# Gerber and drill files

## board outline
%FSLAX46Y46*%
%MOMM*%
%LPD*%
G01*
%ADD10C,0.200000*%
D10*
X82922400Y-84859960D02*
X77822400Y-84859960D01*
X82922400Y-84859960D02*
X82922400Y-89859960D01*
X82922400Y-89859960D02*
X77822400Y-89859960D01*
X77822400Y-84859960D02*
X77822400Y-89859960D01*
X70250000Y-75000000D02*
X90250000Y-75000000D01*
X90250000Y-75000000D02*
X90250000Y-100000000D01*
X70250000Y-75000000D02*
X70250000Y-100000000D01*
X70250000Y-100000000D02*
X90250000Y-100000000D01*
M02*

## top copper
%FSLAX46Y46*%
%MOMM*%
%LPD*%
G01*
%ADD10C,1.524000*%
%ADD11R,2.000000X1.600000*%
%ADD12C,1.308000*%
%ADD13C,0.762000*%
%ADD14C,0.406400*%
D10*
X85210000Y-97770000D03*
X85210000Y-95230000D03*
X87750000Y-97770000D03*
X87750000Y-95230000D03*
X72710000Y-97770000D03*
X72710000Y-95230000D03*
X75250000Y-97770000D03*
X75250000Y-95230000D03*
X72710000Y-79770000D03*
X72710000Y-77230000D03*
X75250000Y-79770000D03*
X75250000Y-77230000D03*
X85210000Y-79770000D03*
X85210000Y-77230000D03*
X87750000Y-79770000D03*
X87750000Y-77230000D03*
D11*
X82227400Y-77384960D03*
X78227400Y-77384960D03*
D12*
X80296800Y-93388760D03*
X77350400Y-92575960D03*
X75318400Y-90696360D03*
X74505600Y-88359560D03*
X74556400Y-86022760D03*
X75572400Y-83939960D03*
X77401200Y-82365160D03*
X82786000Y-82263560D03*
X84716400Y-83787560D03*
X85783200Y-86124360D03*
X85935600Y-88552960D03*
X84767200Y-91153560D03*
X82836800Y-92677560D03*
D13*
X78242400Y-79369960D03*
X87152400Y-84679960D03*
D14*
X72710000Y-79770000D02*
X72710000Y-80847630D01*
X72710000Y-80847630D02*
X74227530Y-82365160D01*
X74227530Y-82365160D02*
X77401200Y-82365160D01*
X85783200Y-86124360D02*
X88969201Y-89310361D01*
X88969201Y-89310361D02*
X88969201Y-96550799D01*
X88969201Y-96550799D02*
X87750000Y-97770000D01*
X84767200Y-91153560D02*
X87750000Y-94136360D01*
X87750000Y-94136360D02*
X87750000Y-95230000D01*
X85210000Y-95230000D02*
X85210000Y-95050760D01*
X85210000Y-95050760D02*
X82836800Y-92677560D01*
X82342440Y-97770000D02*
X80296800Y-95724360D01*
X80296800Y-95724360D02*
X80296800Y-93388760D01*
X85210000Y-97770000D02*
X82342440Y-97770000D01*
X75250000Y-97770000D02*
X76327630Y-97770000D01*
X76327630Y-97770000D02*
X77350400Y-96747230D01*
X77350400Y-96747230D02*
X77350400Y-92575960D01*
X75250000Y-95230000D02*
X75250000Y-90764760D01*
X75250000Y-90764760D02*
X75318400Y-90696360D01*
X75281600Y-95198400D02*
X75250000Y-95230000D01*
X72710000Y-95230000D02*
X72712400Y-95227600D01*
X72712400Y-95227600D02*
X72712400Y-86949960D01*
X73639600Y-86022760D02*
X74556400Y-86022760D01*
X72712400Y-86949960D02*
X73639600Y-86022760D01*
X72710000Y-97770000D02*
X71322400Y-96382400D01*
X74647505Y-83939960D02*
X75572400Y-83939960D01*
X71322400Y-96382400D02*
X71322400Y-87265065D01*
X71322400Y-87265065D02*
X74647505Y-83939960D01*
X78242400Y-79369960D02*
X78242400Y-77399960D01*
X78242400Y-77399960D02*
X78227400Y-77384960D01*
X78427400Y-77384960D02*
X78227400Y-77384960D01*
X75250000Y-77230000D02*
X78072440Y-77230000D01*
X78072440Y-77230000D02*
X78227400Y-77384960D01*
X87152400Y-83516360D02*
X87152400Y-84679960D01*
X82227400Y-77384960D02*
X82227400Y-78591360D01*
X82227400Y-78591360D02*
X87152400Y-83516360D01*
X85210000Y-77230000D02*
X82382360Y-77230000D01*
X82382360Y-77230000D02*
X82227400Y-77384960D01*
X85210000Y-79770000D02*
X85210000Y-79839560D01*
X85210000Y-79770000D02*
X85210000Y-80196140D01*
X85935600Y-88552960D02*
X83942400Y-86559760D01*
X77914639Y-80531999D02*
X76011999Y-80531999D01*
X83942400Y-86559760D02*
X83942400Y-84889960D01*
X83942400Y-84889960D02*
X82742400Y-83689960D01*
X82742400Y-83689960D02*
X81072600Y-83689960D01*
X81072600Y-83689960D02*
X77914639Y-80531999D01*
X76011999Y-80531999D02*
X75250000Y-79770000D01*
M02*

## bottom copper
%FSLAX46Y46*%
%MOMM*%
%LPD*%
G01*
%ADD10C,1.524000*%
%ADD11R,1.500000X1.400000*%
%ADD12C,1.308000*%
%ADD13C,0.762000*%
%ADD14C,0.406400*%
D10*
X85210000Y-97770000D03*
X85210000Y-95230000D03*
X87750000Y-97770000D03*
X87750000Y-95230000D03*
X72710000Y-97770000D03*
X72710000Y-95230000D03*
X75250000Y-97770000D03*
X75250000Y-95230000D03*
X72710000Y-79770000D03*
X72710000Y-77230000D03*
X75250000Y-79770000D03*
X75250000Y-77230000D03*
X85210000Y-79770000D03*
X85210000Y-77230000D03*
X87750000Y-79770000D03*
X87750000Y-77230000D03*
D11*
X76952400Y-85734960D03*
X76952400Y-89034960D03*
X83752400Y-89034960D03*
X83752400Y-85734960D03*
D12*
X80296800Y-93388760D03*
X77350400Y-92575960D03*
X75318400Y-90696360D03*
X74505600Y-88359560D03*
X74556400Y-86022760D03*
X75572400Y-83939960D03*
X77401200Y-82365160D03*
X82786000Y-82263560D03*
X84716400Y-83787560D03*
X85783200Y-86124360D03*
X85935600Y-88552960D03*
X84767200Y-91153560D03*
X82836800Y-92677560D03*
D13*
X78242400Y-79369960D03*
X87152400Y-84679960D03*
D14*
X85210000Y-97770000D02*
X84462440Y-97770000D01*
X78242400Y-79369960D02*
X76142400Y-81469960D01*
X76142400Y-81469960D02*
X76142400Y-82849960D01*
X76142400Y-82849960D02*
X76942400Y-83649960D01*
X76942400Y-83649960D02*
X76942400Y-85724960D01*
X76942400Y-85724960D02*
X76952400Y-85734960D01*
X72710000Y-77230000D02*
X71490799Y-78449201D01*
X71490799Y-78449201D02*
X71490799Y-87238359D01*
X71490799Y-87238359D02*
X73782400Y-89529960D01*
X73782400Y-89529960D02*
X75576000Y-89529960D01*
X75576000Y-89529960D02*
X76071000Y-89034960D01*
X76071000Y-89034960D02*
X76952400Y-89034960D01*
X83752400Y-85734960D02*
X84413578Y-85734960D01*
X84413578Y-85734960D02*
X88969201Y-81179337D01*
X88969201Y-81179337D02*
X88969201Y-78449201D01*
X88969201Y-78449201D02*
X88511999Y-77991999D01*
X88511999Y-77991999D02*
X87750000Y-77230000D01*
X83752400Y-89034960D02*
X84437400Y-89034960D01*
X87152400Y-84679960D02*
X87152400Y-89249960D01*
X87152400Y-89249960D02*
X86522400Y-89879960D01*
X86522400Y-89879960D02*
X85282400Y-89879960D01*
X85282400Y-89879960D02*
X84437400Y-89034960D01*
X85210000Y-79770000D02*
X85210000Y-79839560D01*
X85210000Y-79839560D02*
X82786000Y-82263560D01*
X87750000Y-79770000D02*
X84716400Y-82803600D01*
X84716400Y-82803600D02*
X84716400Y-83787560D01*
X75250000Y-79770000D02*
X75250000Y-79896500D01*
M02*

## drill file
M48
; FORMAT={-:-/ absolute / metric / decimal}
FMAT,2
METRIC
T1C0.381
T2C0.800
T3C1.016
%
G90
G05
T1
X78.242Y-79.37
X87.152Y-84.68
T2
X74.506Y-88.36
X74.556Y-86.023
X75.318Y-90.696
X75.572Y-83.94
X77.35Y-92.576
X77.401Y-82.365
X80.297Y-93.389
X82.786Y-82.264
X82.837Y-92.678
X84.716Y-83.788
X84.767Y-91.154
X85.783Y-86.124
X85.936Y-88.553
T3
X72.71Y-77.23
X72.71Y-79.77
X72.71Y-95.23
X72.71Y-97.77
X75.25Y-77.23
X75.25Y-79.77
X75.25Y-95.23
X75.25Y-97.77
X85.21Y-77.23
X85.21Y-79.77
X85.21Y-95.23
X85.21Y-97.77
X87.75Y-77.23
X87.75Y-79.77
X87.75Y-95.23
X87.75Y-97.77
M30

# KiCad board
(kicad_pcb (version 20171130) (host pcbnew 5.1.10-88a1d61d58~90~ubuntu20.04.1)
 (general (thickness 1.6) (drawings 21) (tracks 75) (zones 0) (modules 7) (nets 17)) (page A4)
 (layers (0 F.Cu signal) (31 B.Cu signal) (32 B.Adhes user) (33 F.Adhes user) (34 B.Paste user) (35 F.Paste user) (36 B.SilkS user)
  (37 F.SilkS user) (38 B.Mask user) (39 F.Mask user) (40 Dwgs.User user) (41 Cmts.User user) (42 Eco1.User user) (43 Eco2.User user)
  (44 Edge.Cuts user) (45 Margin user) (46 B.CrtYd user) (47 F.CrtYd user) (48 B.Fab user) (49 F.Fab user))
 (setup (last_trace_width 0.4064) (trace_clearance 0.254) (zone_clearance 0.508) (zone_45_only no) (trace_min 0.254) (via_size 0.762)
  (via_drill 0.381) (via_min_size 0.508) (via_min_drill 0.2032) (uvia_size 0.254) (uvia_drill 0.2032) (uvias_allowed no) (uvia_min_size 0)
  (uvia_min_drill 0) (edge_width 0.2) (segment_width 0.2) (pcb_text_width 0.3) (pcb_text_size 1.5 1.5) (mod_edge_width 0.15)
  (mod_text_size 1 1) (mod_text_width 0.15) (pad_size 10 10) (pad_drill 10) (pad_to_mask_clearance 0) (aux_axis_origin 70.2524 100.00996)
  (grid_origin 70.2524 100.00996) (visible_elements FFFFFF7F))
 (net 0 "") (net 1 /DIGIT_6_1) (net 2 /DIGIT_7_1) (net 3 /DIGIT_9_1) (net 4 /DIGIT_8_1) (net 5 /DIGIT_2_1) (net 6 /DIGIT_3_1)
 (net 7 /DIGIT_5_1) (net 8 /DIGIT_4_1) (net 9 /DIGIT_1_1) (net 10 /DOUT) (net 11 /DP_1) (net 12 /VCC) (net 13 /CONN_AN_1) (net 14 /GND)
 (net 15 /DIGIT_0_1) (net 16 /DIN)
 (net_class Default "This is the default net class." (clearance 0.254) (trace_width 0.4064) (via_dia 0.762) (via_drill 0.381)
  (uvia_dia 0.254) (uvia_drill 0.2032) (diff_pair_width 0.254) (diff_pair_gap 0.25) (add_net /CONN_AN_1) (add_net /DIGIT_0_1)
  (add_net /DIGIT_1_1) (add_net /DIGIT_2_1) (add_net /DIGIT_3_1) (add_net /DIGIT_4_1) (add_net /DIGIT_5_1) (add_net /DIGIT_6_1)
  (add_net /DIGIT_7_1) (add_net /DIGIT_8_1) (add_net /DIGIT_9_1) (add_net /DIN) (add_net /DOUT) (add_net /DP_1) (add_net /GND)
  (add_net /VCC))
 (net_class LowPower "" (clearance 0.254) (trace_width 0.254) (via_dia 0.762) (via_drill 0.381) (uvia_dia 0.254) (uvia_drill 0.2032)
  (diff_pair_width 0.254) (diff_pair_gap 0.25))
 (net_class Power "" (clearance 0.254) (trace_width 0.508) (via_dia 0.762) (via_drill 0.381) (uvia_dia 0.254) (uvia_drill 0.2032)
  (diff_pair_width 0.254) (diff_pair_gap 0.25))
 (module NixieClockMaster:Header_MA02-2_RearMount (layer F.Cu) (at 87.75 96.5)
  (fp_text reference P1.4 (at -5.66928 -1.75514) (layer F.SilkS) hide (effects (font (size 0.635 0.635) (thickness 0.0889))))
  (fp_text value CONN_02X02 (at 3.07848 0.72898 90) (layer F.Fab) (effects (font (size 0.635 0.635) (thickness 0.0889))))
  (pad 1 thru_hole circle (at -2.54 1.27) (size 1.524 1.524) (drill 1.016) (layers *.Cu *.Mask F.Paste F.SilkS) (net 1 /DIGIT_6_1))
  (pad 2 thru_hole circle (at -2.54 -1.27) (size 1.524 1.524) (drill 1.016) (layers *.Cu *.Mask F.Paste F.SilkS) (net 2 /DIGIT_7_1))
  (pad 3 thru_hole circle (at 0 1.27) (size 1.524 1.524) (drill 1.016) (layers *.Cu *.Mask F.Paste F.SilkS) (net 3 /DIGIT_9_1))
  (pad 4 thru_hole circle (at 0 -1.27) (size 1.524 1.524) (drill 1.016) (layers *.Cu *.Mask F.Paste F.SilkS) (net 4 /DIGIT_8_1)))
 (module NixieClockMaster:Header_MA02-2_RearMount (layer F.Cu) (at 75.25 96.5)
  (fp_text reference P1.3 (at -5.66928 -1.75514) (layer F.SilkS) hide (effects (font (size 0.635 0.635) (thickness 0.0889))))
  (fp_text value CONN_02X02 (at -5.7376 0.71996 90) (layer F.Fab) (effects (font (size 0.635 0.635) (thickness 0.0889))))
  (pad 1 thru_hole circle (at -2.54 1.27) (size 1.524 1.524) (drill 1.016) (layers *.Cu *.Mask F.Paste F.SilkS) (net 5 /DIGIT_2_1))
  (pad 2 thru_hole circle (at -2.54 -1.27) (size 1.524 1.524) (drill 1.016) (layers *.Cu *.Mask F.Paste F.SilkS) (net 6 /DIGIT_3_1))
  (pad 3 thru_hole circle (at 0 1.27) (size 1.524 1.524) (drill 1.016) (layers *.Cu *.Mask F.Paste F.SilkS) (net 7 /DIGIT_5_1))
  (pad 4 thru_hole circle (at 0 -1.27) (size 1.524 1.524) (drill 1.016) (layers *.Cu *.Mask F.Paste F.SilkS) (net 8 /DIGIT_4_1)))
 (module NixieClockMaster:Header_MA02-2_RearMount (layer F.Cu) (at 75.25 78.5)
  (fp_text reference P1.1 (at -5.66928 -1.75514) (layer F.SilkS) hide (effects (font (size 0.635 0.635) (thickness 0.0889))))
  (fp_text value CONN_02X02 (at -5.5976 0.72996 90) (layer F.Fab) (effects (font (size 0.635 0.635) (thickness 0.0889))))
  (pad 1 thru_hole circle (at -2.54 1.27) (size 1.524 1.524) (drill 1.016) (layers *.Cu *.Mask F.Paste F.SilkS) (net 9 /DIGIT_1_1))
  (pad 2 thru_hole circle (at -2.54 -1.27) (size 1.524 1.524) (drill 1.016) (layers *.Cu *.Mask F.Paste F.SilkS) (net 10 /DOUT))
  (pad 3 thru_hole circle (at 0 1.27) (size 1.524 1.524) (drill 1.016) (layers *.Cu *.Mask F.Paste F.SilkS) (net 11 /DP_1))
  (pad 4 thru_hole circle (at 0 -1.27) (size 1.524 1.524) (drill 1.016) (layers *.Cu *.Mask F.Paste F.SilkS) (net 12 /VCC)))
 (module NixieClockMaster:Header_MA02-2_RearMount (layer F.Cu) (at 87.75 78.5)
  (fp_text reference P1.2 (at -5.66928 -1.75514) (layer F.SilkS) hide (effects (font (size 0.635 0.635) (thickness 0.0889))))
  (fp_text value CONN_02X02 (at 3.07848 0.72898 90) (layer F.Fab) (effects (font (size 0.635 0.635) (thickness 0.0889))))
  (pad 1 thru_hole circle (at -2.54 1.27) (size 1.524 1.524) (drill 1.016) (layers *.Cu *.Mask F.Paste F.SilkS) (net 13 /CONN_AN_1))
  (pad 2 thru_hole circle (at -2.54 -1.27) (size 1.524 1.524) (drill 1.016) (layers *.Cu *.Mask F.Paste F.SilkS) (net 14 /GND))
  (pad 3 thru_hole circle (at 0 1.27) (size 1.524 1.524) (drill 1.016) (layers *.Cu *.Mask F.Paste F.SilkS) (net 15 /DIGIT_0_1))
  (pad 4 thru_hole circle (at 0 -1.27) (size 1.524 1.524) (drill 1.016) (layers *.Cu *.Mask F.Paste F.SilkS) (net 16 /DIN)))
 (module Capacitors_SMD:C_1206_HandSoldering (layer F.Cu) (at 80.2274 77.38496 180)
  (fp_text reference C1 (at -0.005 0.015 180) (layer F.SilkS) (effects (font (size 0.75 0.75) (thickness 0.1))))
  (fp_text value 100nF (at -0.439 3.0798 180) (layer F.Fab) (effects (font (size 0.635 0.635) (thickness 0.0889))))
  (pad 1 smd rect (at -2 0 180) (size 2 1.6) (layers F.Cu F.Paste F.Mask) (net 14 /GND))
  (pad 2 smd rect (at 2 0 180) (size 2 1.6) (layers F.Cu F.Paste F.Mask) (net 12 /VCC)))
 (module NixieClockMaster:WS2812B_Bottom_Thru (layer F.Cu) (at 80.3524 87.38496 90)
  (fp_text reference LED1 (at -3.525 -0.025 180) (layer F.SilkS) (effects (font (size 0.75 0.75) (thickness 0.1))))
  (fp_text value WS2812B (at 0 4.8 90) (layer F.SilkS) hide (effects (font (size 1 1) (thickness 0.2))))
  (pad 1 smd rect (at 1.65 -3.4 90) (size 1.4 1.5) (layers B.Cu B.Paste B.Mask) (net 12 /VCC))
  (pad 2 smd rect (at -1.65 -3.4 90) (size 1.4 1.5) (layers B.Cu B.Paste B.Mask) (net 10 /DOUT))
  (pad 3 smd rect (at -1.65 3.4 90) (size 1.4 1.5) (layers B.Cu B.Paste B.Mask) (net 14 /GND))
  (pad 4 smd rect (at 1.65 3.4 90) (size 1.4 1.5) (layers B.Cu B.Paste B.Mask) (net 16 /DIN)))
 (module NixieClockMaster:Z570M (layer F.Cu) (at 80.1952 87.49596 180)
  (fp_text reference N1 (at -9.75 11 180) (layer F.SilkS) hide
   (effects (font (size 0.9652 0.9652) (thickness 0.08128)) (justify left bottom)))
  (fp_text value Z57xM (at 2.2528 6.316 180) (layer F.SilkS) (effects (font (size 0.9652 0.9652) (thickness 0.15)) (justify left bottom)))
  (pad 6 thru_hole circle (at -0.1016 -5.8928 180) (size 1.308 1.308) (drill 0.8) (layers *.Cu *.Mask) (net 1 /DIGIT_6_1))
  (pad 5 thru_hole circle (at 2.8448 -5.08 180) (size 1.308 1.308) (drill 0.8) (layers *.Cu *.Mask) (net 7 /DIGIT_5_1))
  (pad 4 thru_hole circle (at 4.8768 -3.2004 180) (size 1.308 1.308) (drill 0.8) (layers *.Cu *.Mask) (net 8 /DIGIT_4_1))
  (pad N/C thru_hole circle (at 5.6896 -0.8636 180) (size 1.308 1.308) (drill 0.8) (layers *.Cu *.Mask))
  (pad 3 thru_hole circle (at 5.6388 1.4732 180) (size 1.308 1.308) (drill 0.8) (layers *.Cu *.Mask) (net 6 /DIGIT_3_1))
  (pad 2 thru_hole circle (at 4.6228 3.556 180) (size 1.308 1.308) (drill 0.8) (layers *.Cu *.Mask) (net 5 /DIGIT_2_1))
  (pad 1 thru_hole circle (at 2.794 5.1308 180) (size 1.308 1.308) (drill 0.8) (layers *.Cu *.Mask) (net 9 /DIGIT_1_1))
  (pad A thru_hole circle (at -2.5908 5.2324 180) (size 1.308 1.308) (drill 0.8) (layers *.Cu *.Mask) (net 13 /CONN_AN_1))
  (pad 0 thru_hole circle (at -4.5212 3.7084 180) (size 1.308 1.308) (drill 0.8) (layers *.Cu *.Mask) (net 15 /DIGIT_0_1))
  (pad 9 thru_hole circle (at -5.588 1.3716 180) (size 1.308 1.308) (drill 0.8) (layers *.Cu *.Mask) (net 3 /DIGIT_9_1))
  (pad RHDP thru_hole circle (at -5.7404 -1.057 180) (size 1.308 1.308) (drill 0.8) (layers *.Cu *.Mask) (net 11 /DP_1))
  (pad 8 thru_hole circle (at -4.572 -3.6576 180) (size 1.308 1.308) (drill 0.8) (layers *.Cu *.Mask) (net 4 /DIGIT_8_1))
  (pad 7 thru_hole circle (at -2.6416 -5.1816 180) (size 1.308 1.308) (drill 0.8) (layers *.Cu *.Mask) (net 2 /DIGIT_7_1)))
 (gr_line (start 82.9224 84.85996) (end 77.8224 84.85996) (layer Edge.Cuts) (width 0.2))
 (gr_line (start 82.9224 84.85996) (end 82.9224 89.85996) (layer Edge.Cuts) (width 0.2))
 (gr_line (start 82.9224 89.85996) (end 77.8224 89.85996) (layer Edge.Cuts) (width 0.2))
 (gr_line (start 77.8224 84.85996) (end 77.8224 89.85996) (layer Edge.Cuts) (width 0.2))
 (gr_line (start 70.25 75) (end 90.25 75) (layer Edge.Cuts) (width 0.2))
 (gr_line (start 90.25 75) (end 90.25 100) (layer Edge.Cuts) (width 0.2))
 (gr_line (start 70.25 75) (end 70.25 100) (layer Edge.Cuts) (width 0.2))
 (gr_line (start 70.25 100) (end 90.25 100) (layer Edge.Cuts) (width 0.2))
 (segment (start 72.71 79.77) (end 72.71 80.84763) (width 0.4064) (layer F.Cu) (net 9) (status 10))
 (segment (start 72.71 80.84763) (end 74.22753 82.36516) (width 0.4064) (layer F.Cu) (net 9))
 (segment (start 74.22753 82.36516) (end 77.4012 82.36516) (width 0.4064) (layer F.Cu) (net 9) (status 20))
 (segment (start 85.7832 86.12436) (end 88.969201 89.310361) (width 0.4064) (layer F.Cu) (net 3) (status 10))
 (segment (start 88.969201 89.310361) (end 88.969201 96.550799) (width 0.4064) (layer F.Cu) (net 3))
 (segment (start 88.969201 96.550799) (end 87.75 97.77) (width 0.4064) (layer F.Cu) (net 3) (status 20))
 (segment (start 84.7672 91.15356) (end 87.75 94.13636) (width 0.4064) (layer F.Cu) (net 4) (status 10))
 (segment (start 87.75 94.13636) (end 87.75 95.23) (width 0.4064) (layer F.Cu) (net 4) (status 20))
 (segment (start 85.21 95.23) (end 85.21 95.05076) (width 0.4064) (layer F.Cu) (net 2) (status 30))
 (segment (start 85.21 95.05076) (end 82.8368 92.67756) (width 0.4064) (layer F.Cu) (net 2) (status 30))
 (segment (start 82.34244 97.77) (end 80.2968 95.72436) (width 0.4064) (layer F.Cu) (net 1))
 (segment (start 80.2968 95.72436) (end 80.2968 93.38876) (width 0.4064) (layer F.Cu) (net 1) (status 20))
 (segment (start 85.21 97.77) (end 82.34244 97.77) (width 0.4064) (layer F.Cu) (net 1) (status 10))
 (segment (start 85.21 97.77) (end 84.46244 97.77) (width 0.4064) (layer B.Cu) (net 1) (status 30))
 (segment (start 75.25 97.77) (end 76.32763 97.77) (width 0.4064) (layer F.Cu) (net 7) (status 10))
 (segment (start 76.32763 97.77) (end 77.3504 96.74723) (width 0.4064) (layer F.Cu) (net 7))
 (segment (start 77.3504 96.74723) (end 77.3504 92.57596) (width 0.4064) (layer F.Cu) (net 7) (status 20))
 (segment (start 75.25 95.23) (end 75.25 90.76476) (width 0.4064) (layer F.Cu) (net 8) (status 30))
 (segment (start 75.25 90.76476) (end 75.3184 90.69636) (width 0.4064) (layer F.Cu) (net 8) (status 30))
 (segment (start 75.2816 95.1984) (end 75.25 95.23) (width 0.4064) (layer F.Cu) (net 8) (status 30))
 (segment (start 72.71 95.23) (end 72.7124 95.2276) (width 0.4064) (layer F.Cu) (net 6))
 (segment (start 72.7124 95.2276) (end 72.7124 86.94996) (width 0.4064) (layer F.Cu) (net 6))
 (segment (start 73.6396 86.02276) (end 74.5564 86.02276) (width 0.4064) (layer F.Cu) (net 6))
 (segment (start 72.7124 86.94996) (end 73.6396 86.02276) (width 0.4064) (layer F.Cu) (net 6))
 (segment (start 72.71 97.77) (end 71.3224 96.3824) (width 0.4064) (layer F.Cu) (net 5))
 (segment (start 74.647505 83.93996) (end 75.5724 83.93996) (width 0.4064) (layer F.Cu) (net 5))
 (segment (start 71.3224 96.3824) (end 71.3224 87.265065) (width 0.4064) (layer F.Cu) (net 5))
 (segment (start 71.3224 87.265065) (end 74.647505 83.93996) (width 0.4064) (layer F.Cu) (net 5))
 (segment (start 78.2424 79.36996) (end 76.1424 81.46996) (width 0.4064) (layer B.Cu) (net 12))
 (segment (start 76.1424 81.46996) (end 76.1424 82.84996) (width 0.4064) (layer B.Cu) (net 12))
 (segment (start 76.1424 82.84996) (end 76.9424 83.64996) (width 0.4064) (layer B.Cu) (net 12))
 (segment (start 76.9424 83.64996) (end 76.9424 85.72496) (width 0.4064) (layer B.Cu) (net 12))
 (segment (start 76.9424 85.72496) (end 76.9524 85.73496) (width 0.4064) (layer B.Cu) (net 12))
 (segment (start 78.2424 79.36996) (end 78.2424 77.39996) (width 0.4064) (layer F.Cu) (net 12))
 (segment (start 78.2424 77.39996) (end 78.2274 77.38496) (width 0.4064) (layer F.Cu) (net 12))
 (via (at 78.2424 79.36996) (size 0.762) (drill 0.381) (layers F.Cu B.Cu) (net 12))
 (segment (start 78.4274 77.38496) (end 78.2274 77.38496) (width 0.4064) (layer F.Cu) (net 12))
 (segment (start 75.25 77.23) (end 78.07244 77.23) (width 0.4064) (layer F.Cu) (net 12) (status 30))
 (segment (start 78.07244 77.23) (end 78.2274 77.38496) (width 0.4064) (layer F.Cu) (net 12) (status 30))
 (segment (start 72.71 77.23) (end 71.490799 78.449201) (width 0.4064) (layer B.Cu) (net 10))
 (segment (start 71.490799 78.449201) (end 71.490799 87.238359) (width 0.4064) (layer B.Cu) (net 10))
 (segment (start 71.490799 87.238359) (end 73.7824 89.52996) (width 0.4064) (layer B.Cu) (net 10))
 (segment (start 73.7824 89.52996) (end 75.576 89.52996) (width 0.4064) (layer B.Cu) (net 10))
 (segment (start 75.576 89.52996) (end 76.071 89.03496) (width 0.4064) (layer B.Cu) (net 10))
 (segment (start 76.071 89.03496) (end 76.9524 89.03496) (width 0.4064) (layer B.Cu) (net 10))
 (segment (start 83.7524 85.73496) (end 84.413578 85.73496) (width 0.4064) (layer B.Cu) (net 16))
 (segment (start 84.413578 85.73496) (end 88.969201 81.179337) (width 0.4064) (layer B.Cu) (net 16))
 (segment (start 88.969201 81.179337) (end 88.969201 78.449201) (width 0.4064) (layer B.Cu) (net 16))
 (segment (start 88.969201 78.449201) (end 88.511999 77.991999) (width 0.4064) (layer B.Cu) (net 16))
 (segment (start 88.511999 77.991999) (end 87.75 77.23) (width 0.4064) (layer B.Cu) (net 16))
 (segment (start 83.7524 89.03496) (end 84.4374 89.03496) (width 0.4064) (layer B.Cu) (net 14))
 (segment (start 87.1524 84.67996) (end 87.1524 89.24996) (width 0.4064) (layer B.Cu) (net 14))
 (segment (start 87.1524 89.24996) (end 86.5224 89.87996) (width 0.4064) (layer B.Cu) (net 14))
 (segment (start 86.5224 89.87996) (end 85.2824 89.87996) (width 0.4064) (layer B.Cu) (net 14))
 (segment (start 85.2824 89.87996) (end 84.4374 89.03496) (width 0.4064) (layer B.Cu) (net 14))
 (segment (start 87.1524 83.51636) (end 87.1524 84.67996) (width 0.4064) (layer F.Cu) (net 14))
 (via (at 87.1524 84.67996) (size 0.762) (drill 0.381) (layers F.Cu B.Cu) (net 14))
 (segment (start 82.2274 77.38496) (end 82.2274 78.59136) (width 0.4064) (layer F.Cu) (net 14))
 (segment (start 82.2274 78.59136) (end 87.1524 83.51636) (width 0.4064) (layer F.Cu) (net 14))
 (segment (start 85.21 77.23) (end 82.38236 77.23) (width 0.4064) (layer F.Cu) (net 14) (status 30))
 (segment (start 82.38236 77.23) (end 82.2274 77.38496) (width 0.4064) (layer F.Cu) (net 14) (status 30))
 (segment (start 85.21 79.77) (end 85.21 79.83956) (width 0.4064) (layer B.Cu) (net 13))
 (segment (start 85.21 79.83956) (end 82.786 82.26356) (width 0.4064) (layer B.Cu) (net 13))
 (segment (start 85.21 79.77) (end 85.21 79.83956) (width 0.4064) (layer F.Cu) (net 13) (status 30))
 (segment (start 85.21 79.77) (end 85.21 80.19614) (width 0.4064) (layer F.Cu) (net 13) (status 30))
 (segment (start 87.75 79.77) (end 84.7164 82.8036) (width 0.4064) (layer B.Cu) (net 15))
 (segment (start 84.7164 82.8036) (end 84.7164 83.78756) (width 0.4064) (layer B.Cu) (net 15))
 (segment (start 85.9356 88.55296) (end 83.9424 86.55976) (width 0.4064) (layer F.Cu) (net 11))
 (segment (start 77.914639 80.531999) (end 76.011999 80.531999) (width 0.4064) (layer F.Cu) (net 11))
 (segment (start 83.9424 86.55976) (end 83.9424 84.88996) (width 0.4064) (layer F.Cu) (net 11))
 (segment (start 83.9424 84.88996) (end 82.7424 83.68996) (width 0.4064) (layer F.Cu) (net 11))
 (segment (start 82.7424 83.68996) (end 81.0726 83.68996) (width 0.4064) (layer F.Cu) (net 11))
 (segment (start 81.0726 83.68996) (end 77.914639 80.531999) (width 0.4064) (layer F.Cu) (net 11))
 (segment (start 76.011999 80.531999) (end 75.25 79.77) (width 0.4064) (layer F.Cu) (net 11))
 (segment (start 75.25 79.77) (end 75.25 79.8965) (width 0.4064) (layer B.Cu) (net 11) (status 30)))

